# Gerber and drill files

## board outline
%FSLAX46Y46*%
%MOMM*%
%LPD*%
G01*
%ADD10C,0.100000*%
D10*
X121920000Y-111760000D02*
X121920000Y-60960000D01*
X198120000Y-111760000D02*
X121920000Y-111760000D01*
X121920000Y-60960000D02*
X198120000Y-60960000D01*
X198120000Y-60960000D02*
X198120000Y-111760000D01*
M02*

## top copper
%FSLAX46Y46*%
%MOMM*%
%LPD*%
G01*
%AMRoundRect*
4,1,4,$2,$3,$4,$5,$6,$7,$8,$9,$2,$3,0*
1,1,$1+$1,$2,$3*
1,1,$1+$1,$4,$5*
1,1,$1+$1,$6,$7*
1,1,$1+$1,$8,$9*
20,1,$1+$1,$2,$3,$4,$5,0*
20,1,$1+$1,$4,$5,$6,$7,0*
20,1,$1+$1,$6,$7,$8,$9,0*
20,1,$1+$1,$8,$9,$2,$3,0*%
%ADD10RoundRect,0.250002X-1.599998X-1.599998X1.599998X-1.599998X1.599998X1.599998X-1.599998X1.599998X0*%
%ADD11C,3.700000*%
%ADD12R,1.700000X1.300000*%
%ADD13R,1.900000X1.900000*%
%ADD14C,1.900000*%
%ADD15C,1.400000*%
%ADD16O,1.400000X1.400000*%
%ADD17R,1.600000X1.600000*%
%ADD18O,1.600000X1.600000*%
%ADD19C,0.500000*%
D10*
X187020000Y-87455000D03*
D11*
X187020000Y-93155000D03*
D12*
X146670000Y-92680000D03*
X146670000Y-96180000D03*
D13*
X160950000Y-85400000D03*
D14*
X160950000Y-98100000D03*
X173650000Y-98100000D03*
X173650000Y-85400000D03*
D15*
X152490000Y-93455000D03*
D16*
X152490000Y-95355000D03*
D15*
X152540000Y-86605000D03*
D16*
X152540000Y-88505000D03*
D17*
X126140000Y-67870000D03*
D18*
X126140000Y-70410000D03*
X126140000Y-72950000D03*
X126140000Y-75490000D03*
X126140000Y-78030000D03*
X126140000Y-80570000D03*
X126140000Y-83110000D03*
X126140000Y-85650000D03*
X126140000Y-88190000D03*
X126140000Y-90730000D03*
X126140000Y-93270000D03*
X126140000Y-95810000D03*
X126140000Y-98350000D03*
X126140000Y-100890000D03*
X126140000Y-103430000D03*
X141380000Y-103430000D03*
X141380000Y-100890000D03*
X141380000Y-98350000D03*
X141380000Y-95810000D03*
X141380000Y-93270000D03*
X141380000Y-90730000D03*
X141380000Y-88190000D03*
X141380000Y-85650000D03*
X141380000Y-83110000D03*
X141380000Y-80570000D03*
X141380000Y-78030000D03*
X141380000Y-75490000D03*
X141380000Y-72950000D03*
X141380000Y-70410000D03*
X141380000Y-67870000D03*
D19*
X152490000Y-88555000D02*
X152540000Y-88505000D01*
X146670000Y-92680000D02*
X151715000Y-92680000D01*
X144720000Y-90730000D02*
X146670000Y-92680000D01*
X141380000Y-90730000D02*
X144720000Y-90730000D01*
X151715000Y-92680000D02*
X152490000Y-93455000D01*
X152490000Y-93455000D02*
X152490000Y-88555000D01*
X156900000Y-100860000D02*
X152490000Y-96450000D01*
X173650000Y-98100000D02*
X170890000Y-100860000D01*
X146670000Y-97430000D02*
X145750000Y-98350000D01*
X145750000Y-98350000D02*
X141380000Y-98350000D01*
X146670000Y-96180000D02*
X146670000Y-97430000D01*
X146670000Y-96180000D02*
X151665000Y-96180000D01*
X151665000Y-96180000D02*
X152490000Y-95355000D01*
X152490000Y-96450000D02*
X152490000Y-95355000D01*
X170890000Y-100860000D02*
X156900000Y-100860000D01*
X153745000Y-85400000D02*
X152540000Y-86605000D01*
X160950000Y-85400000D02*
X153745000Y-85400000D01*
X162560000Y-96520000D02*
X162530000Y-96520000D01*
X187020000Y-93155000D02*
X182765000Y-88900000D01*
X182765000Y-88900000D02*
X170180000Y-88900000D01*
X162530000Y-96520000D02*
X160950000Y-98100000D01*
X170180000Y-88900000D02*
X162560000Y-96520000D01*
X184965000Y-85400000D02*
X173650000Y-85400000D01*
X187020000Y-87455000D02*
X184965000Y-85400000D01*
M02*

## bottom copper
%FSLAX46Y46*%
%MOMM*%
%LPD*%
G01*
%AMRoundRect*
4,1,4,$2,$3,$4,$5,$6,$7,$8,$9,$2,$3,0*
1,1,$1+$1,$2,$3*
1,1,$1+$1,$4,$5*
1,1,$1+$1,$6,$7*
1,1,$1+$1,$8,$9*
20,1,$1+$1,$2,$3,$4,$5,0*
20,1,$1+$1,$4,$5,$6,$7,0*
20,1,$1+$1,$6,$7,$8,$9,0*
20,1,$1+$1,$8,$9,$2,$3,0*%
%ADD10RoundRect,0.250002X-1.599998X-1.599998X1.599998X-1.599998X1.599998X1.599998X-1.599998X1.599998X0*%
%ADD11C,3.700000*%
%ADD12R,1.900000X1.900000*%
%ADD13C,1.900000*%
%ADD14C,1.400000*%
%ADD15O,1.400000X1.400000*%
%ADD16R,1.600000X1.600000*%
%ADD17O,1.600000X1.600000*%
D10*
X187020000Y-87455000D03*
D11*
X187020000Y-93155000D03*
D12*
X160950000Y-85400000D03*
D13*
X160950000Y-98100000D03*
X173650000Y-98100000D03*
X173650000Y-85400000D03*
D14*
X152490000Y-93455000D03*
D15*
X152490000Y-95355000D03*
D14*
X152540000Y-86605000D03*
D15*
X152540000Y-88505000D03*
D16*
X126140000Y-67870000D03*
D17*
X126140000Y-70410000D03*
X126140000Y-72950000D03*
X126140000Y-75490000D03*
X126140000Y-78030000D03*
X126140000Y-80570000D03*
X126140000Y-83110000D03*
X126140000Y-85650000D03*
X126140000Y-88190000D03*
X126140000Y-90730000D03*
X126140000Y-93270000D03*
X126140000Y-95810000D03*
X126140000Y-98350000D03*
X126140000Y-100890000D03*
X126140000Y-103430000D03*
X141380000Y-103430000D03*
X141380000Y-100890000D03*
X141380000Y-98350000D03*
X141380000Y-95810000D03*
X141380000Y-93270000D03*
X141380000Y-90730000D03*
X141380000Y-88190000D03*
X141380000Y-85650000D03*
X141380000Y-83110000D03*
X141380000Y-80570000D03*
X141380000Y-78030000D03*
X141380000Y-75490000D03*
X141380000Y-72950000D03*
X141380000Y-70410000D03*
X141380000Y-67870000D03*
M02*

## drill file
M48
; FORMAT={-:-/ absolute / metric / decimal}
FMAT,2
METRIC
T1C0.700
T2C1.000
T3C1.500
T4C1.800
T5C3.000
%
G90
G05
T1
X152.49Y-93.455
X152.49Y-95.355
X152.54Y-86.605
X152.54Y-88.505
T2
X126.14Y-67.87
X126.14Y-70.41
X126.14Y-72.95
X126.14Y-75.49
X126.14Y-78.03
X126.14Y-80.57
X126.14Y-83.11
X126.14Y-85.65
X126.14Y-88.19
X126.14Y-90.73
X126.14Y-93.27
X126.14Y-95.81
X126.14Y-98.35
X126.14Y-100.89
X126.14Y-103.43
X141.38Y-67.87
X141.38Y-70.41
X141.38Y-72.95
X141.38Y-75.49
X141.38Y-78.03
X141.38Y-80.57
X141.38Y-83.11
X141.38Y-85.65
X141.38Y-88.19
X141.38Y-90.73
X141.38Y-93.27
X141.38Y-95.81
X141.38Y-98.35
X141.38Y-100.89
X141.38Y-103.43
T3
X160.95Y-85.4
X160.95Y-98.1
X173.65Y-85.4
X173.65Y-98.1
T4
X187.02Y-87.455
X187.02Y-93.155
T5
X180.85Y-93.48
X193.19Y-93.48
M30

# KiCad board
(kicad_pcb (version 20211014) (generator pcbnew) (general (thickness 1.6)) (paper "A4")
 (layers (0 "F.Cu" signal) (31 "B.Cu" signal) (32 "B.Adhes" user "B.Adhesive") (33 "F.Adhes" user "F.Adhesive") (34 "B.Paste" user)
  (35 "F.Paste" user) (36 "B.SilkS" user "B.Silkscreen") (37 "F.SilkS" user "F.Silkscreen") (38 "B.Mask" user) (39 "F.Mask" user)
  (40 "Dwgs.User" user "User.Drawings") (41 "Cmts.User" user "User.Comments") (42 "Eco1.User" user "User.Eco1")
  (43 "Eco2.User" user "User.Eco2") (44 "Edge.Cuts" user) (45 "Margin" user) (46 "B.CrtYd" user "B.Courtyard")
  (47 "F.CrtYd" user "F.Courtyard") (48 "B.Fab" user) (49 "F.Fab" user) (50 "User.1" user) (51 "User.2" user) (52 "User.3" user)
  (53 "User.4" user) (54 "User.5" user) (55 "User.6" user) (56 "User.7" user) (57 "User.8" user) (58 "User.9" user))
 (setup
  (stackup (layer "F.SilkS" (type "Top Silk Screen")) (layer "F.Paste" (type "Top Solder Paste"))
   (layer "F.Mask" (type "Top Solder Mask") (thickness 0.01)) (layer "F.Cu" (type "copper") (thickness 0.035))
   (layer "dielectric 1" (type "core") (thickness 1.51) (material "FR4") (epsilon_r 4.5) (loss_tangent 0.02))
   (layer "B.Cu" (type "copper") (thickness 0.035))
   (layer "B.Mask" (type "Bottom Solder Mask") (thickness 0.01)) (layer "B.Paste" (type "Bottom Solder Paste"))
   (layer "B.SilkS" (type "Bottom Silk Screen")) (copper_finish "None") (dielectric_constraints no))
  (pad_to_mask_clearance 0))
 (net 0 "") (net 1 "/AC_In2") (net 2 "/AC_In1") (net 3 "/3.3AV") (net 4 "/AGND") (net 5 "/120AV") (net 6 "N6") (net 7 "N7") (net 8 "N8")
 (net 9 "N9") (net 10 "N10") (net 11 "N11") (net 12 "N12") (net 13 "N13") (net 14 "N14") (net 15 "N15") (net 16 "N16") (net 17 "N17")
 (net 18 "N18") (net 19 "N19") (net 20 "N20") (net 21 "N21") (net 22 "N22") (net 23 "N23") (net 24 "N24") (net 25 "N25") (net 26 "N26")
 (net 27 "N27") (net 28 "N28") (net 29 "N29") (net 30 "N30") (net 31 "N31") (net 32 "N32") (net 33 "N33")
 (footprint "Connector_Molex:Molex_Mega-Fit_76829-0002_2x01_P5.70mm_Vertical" (layer "F.Cu") (at 187.02 87.455)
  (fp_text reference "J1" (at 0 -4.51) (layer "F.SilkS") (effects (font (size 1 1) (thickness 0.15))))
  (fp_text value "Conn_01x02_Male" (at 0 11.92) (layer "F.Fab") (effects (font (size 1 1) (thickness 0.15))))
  (pad "" np_thru_hole circle locked (at -6.17 6.025) (size 3 3) (drill 3) (layers *.Cu *.Mask))
  (pad "" np_thru_hole circle locked (at 6.17 6.025) (size 3 3) (drill 3) (layers *.Cu *.Mask))
  (pad "1" thru_hole roundrect locked (at 0 0) (size 3.7 3.7) (drill 1.8) (layers *.Cu *.Mask) (roundrect_rratio 0.06756810811)
   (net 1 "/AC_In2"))
  (pad "2" thru_hole circle locked (at 0 5.7) (size 3.7 3.7) (drill 1.8) (layers *.Cu *.Mask) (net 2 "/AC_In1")))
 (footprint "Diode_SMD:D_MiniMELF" (layer "F.Cu") (at 146.67 94.43 -90)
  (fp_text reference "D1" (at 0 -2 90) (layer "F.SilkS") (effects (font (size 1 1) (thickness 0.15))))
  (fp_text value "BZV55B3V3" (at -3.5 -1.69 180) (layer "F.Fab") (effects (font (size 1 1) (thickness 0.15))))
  (pad "1" smd rect locked (at -1.75 0 270) (size 1.3 1.7) (layers "F.Cu" "F.Paste" "F.Mask") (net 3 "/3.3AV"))
  (pad "2" smd rect locked (at 1.75 0 270) (size 1.3 1.7) (layers "F.Cu" "F.Paste" "F.Mask") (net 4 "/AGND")))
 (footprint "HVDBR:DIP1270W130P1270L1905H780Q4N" (layer "F.Cu") (at 167.3 91.75)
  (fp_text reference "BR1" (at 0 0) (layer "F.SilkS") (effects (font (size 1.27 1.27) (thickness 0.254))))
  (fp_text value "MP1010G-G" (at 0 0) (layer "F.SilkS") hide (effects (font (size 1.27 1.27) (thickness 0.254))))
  (pad "1" thru_hole rect locked (at -6.35 -6.35) (size 1.9 1.9) (drill 1.5) (layers *.Cu *.Mask) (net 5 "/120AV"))
  (pad "2" thru_hole circle locked (at -6.35 6.35) (size 1.9 1.9) (drill 1.5) (layers *.Cu *.Mask) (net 2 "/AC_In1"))
  (pad "3" thru_hole circle locked (at 6.35 6.35) (size 1.9 1.9) (drill 1.5) (layers *.Cu *.Mask) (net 4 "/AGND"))
  (pad "4" thru_hole circle locked (at 6.35 -6.35) (size 1.9 1.9) (drill 1.5) (layers *.Cu *.Mask) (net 1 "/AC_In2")))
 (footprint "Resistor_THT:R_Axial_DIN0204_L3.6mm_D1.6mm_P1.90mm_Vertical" (layer "F.Cu") (at 152.49 93.455 -90)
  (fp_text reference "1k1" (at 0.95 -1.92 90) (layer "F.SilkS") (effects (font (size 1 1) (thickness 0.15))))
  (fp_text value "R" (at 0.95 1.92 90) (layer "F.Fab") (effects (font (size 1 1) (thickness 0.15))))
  (pad "1" thru_hole circle locked (at 0 0 270) (size 1.4 1.4) (drill 0.7) (layers *.Cu *.Mask) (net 3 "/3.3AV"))
  (pad "2" thru_hole oval locked (at 1.9 0 270) (size 1.4 1.4) (drill 0.7) (layers *.Cu *.Mask) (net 4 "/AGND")))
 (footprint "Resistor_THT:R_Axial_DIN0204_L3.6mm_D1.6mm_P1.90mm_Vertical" (layer "F.Cu") (at 152.54 86.605 -90)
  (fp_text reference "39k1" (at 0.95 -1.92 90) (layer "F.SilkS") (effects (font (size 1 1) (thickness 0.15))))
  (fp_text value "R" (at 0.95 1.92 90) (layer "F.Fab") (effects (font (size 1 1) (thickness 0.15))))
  (pad "1" thru_hole circle locked (at 0 0 270) (size 1.4 1.4) (drill 0.7) (layers *.Cu *.Mask) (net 5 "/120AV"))
  (pad "2" thru_hole oval locked (at 1.9 0 270) (size 1.4 1.4) (drill 0.7) (layers *.Cu *.Mask) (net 3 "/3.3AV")))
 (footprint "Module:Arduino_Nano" (layer "F.Cu") (at 126.14 67.87)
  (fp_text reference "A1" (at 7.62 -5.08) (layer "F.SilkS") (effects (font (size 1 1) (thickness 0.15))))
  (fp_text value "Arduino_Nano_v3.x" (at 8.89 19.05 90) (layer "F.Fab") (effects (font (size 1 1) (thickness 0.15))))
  (pad "1" thru_hole rect locked (at 0 0) (size 1.6 1.6) (drill 1) (layers *.Cu *.Mask) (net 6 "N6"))
  (pad "2" thru_hole oval locked (at 0 2.54) (size 1.6 1.6) (drill 1) (layers *.Cu *.Mask) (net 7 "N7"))
  (pad "3" thru_hole oval locked (at 0 5.08) (size 1.6 1.6) (drill 1) (layers *.Cu *.Mask) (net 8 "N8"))
  (pad "4" thru_hole oval locked (at 0 7.62) (size 1.6 1.6) (drill 1) (layers *.Cu *.Mask) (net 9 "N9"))
  (pad "5" thru_hole oval locked (at 0 10.16) (size 1.6 1.6) (drill 1) (layers *.Cu *.Mask) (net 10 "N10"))
  (pad "6" thru_hole oval locked (at 0 12.7) (size 1.6 1.6) (drill 1) (layers *.Cu *.Mask) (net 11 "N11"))
  (pad "7" thru_hole oval locked (at 0 15.24) (size 1.6 1.6) (drill 1) (layers *.Cu *.Mask) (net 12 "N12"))
  (pad "8" thru_hole oval locked (at 0 17.78) (size 1.6 1.6) (drill 1) (layers *.Cu *.Mask) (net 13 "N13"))
  (pad "9" thru_hole oval locked (at 0 20.32) (size 1.6 1.6) (drill 1) (layers *.Cu *.Mask) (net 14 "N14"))
  (pad "10" thru_hole oval locked (at 0 22.86) (size 1.6 1.6) (drill 1) (layers *.Cu *.Mask) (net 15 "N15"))
  (pad "11" thru_hole oval locked (at 0 25.4) (size 1.6 1.6) (drill 1) (layers *.Cu *.Mask) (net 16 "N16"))
  (pad "12" thru_hole oval locked (at 0 27.94) (size 1.6 1.6) (drill 1) (layers *.Cu *.Mask) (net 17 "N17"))
  (pad "13" thru_hole oval locked (at 0 30.48) (size 1.6 1.6) (drill 1) (layers *.Cu *.Mask) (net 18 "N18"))
  (pad "14" thru_hole oval locked (at 0 33.02) (size 1.6 1.6) (drill 1) (layers *.Cu *.Mask) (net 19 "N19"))
  (pad "15" thru_hole oval locked (at 0 35.56) (size 1.6 1.6) (drill 1) (layers *.Cu *.Mask) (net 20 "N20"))
  (pad "16" thru_hole oval locked (at 15.24 35.56) (size 1.6 1.6) (drill 1) (layers *.Cu *.Mask) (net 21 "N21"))
  (pad "17" thru_hole oval locked (at 15.24 33.02) (size 1.6 1.6) (drill 1) (layers *.Cu *.Mask) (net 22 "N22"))
  (pad "18" thru_hole oval locked (at 15.24 30.48) (size 1.6 1.6) (drill 1) (layers *.Cu *.Mask) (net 4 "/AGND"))
  (pad "19" thru_hole oval locked (at 15.24 27.94) (size 1.6 1.6) (drill 1) (layers *.Cu *.Mask) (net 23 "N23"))
  (pad "20" thru_hole oval locked (at 15.24 25.4) (size 1.6 1.6) (drill 1) (layers *.Cu *.Mask) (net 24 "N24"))
  (pad "21" thru_hole oval locked (at 15.24 22.86) (size 1.6 1.6) (drill 1) (layers *.Cu *.Mask) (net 3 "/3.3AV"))
  (pad "22" thru_hole oval locked (at 15.24 20.32) (size 1.6 1.6) (drill 1) (layers *.Cu *.Mask) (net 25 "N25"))
  (pad "23" thru_hole oval locked (at 15.24 17.78) (size 1.6 1.6) (drill 1) (layers *.Cu *.Mask) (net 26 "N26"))
  (pad "24" thru_hole oval locked (at 15.24 15.24) (size 1.6 1.6) (drill 1) (layers *.Cu *.Mask) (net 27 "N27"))
  (pad "25" thru_hole oval locked (at 15.24 12.7) (size 1.6 1.6) (drill 1) (layers *.Cu *.Mask) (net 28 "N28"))
  (pad "26" thru_hole oval locked (at 15.24 10.16) (size 1.6 1.6) (drill 1) (layers *.Cu *.Mask) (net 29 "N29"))
  (pad "27" thru_hole oval locked (at 15.24 7.62) (size 1.6 1.6) (drill 1) (layers *.Cu *.Mask) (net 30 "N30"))
  (pad "28" thru_hole oval locked (at 15.24 5.08) (size 1.6 1.6) (drill 1) (layers *.Cu *.Mask) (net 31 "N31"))
  (pad "29" thru_hole oval locked (at 15.24 2.54) (size 1.6 1.6) (drill 1) (layers *.Cu *.Mask) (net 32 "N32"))
  (pad "30" thru_hole oval locked (at 15.24 0) (size 1.6 1.6) (drill 1) (layers *.Cu *.Mask) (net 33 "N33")))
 (gr_line (start 121.92 111.76) (end 121.92 60.96) (layer "Edge.Cuts") (width 0.1))
 (gr_line (start 198.12 111.76) (end 121.92 111.76) (layer "Edge.Cuts") (width 0.1))
 (gr_line (start 121.92 60.96) (end 198.12 60.96) (layer "Edge.Cuts") (width 0.1))
 (gr_line (start 198.12 60.96) (end 198.12 111.76) (layer "Edge.Cuts") (width 0.1))
 (segment (start 152.49 88.555) (end 152.54 88.505) (width 0.5) (layer "F.Cu") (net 3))
 (segment (start 146.67 92.68) (end 151.715 92.68) (width 0.5) (layer "F.Cu") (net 3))
 (segment (start 144.72 90.73) (end 146.67 92.68) (width 0.5) (layer "F.Cu") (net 3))
 (segment (start 141.38 90.73) (end 144.72 90.73) (width 0.5) (layer "F.Cu") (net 3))
 (segment (start 151.715 92.68) (end 152.49 93.455) (width 0.5) (layer "F.Cu") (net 3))
 (segment (start 152.49 93.455) (end 152.49 88.555) (width 0.5) (layer "F.Cu") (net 3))
 (segment (start 156.9 100.86) (end 152.49 96.45) (width 0.5) (layer "F.Cu") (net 4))
 (segment (start 173.65 98.1) (end 170.89 100.86) (width 0.5) (layer "F.Cu") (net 4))
 (segment (start 146.67 97.43) (end 145.75 98.35) (width 0.5) (layer "F.Cu") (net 4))
 (segment (start 145.75 98.35) (end 141.38 98.35) (width 0.5) (layer "F.Cu") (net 4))
 (segment (start 146.67 96.18) (end 146.67 97.43) (width 0.5) (layer "F.Cu") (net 4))
 (segment (start 146.67 96.18) (end 151.665 96.18) (width 0.5) (layer "F.Cu") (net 4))
 (segment (start 151.665 96.18) (end 152.49 95.355) (width 0.5) (layer "F.Cu") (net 4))
 (segment (start 152.49 96.45) (end 152.49 95.355) (width 0.5) (layer "F.Cu") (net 4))
 (segment (start 170.89 100.86) (end 156.9 100.86) (width 0.5) (layer "F.Cu") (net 4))
 (segment (start 153.745 85.4) (end 152.54 86.605) (width 0.5) (layer "F.Cu") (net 5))
 (segment (start 160.95 85.4) (end 153.745 85.4) (width 0.5) (layer "F.Cu") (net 5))
 (segment (start 162.56 96.52) (end 162.53 96.52) (width 0.5) (layer "F.Cu") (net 2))
 (segment (start 187.02 93.155) (end 182.765 88.9) (width 0.5) (layer "F.Cu") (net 2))
 (segment (start 182.765 88.9) (end 170.18 88.9) (width 0.5) (layer "F.Cu") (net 2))
 (segment (start 162.53 96.52) (end 160.95 98.1) (width 0.5) (layer "F.Cu") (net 2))
 (segment (start 170.18 88.9) (end 162.56 96.52) (width 0.5) (layer "F.Cu") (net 2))
 (segment (start 184.965 85.4) (end 173.65 85.4) (width 0.5) (layer "F.Cu") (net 1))
 (segment (start 187.02 87.455) (end 184.965 85.4) (width 0.5) (layer "F.Cu") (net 1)))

